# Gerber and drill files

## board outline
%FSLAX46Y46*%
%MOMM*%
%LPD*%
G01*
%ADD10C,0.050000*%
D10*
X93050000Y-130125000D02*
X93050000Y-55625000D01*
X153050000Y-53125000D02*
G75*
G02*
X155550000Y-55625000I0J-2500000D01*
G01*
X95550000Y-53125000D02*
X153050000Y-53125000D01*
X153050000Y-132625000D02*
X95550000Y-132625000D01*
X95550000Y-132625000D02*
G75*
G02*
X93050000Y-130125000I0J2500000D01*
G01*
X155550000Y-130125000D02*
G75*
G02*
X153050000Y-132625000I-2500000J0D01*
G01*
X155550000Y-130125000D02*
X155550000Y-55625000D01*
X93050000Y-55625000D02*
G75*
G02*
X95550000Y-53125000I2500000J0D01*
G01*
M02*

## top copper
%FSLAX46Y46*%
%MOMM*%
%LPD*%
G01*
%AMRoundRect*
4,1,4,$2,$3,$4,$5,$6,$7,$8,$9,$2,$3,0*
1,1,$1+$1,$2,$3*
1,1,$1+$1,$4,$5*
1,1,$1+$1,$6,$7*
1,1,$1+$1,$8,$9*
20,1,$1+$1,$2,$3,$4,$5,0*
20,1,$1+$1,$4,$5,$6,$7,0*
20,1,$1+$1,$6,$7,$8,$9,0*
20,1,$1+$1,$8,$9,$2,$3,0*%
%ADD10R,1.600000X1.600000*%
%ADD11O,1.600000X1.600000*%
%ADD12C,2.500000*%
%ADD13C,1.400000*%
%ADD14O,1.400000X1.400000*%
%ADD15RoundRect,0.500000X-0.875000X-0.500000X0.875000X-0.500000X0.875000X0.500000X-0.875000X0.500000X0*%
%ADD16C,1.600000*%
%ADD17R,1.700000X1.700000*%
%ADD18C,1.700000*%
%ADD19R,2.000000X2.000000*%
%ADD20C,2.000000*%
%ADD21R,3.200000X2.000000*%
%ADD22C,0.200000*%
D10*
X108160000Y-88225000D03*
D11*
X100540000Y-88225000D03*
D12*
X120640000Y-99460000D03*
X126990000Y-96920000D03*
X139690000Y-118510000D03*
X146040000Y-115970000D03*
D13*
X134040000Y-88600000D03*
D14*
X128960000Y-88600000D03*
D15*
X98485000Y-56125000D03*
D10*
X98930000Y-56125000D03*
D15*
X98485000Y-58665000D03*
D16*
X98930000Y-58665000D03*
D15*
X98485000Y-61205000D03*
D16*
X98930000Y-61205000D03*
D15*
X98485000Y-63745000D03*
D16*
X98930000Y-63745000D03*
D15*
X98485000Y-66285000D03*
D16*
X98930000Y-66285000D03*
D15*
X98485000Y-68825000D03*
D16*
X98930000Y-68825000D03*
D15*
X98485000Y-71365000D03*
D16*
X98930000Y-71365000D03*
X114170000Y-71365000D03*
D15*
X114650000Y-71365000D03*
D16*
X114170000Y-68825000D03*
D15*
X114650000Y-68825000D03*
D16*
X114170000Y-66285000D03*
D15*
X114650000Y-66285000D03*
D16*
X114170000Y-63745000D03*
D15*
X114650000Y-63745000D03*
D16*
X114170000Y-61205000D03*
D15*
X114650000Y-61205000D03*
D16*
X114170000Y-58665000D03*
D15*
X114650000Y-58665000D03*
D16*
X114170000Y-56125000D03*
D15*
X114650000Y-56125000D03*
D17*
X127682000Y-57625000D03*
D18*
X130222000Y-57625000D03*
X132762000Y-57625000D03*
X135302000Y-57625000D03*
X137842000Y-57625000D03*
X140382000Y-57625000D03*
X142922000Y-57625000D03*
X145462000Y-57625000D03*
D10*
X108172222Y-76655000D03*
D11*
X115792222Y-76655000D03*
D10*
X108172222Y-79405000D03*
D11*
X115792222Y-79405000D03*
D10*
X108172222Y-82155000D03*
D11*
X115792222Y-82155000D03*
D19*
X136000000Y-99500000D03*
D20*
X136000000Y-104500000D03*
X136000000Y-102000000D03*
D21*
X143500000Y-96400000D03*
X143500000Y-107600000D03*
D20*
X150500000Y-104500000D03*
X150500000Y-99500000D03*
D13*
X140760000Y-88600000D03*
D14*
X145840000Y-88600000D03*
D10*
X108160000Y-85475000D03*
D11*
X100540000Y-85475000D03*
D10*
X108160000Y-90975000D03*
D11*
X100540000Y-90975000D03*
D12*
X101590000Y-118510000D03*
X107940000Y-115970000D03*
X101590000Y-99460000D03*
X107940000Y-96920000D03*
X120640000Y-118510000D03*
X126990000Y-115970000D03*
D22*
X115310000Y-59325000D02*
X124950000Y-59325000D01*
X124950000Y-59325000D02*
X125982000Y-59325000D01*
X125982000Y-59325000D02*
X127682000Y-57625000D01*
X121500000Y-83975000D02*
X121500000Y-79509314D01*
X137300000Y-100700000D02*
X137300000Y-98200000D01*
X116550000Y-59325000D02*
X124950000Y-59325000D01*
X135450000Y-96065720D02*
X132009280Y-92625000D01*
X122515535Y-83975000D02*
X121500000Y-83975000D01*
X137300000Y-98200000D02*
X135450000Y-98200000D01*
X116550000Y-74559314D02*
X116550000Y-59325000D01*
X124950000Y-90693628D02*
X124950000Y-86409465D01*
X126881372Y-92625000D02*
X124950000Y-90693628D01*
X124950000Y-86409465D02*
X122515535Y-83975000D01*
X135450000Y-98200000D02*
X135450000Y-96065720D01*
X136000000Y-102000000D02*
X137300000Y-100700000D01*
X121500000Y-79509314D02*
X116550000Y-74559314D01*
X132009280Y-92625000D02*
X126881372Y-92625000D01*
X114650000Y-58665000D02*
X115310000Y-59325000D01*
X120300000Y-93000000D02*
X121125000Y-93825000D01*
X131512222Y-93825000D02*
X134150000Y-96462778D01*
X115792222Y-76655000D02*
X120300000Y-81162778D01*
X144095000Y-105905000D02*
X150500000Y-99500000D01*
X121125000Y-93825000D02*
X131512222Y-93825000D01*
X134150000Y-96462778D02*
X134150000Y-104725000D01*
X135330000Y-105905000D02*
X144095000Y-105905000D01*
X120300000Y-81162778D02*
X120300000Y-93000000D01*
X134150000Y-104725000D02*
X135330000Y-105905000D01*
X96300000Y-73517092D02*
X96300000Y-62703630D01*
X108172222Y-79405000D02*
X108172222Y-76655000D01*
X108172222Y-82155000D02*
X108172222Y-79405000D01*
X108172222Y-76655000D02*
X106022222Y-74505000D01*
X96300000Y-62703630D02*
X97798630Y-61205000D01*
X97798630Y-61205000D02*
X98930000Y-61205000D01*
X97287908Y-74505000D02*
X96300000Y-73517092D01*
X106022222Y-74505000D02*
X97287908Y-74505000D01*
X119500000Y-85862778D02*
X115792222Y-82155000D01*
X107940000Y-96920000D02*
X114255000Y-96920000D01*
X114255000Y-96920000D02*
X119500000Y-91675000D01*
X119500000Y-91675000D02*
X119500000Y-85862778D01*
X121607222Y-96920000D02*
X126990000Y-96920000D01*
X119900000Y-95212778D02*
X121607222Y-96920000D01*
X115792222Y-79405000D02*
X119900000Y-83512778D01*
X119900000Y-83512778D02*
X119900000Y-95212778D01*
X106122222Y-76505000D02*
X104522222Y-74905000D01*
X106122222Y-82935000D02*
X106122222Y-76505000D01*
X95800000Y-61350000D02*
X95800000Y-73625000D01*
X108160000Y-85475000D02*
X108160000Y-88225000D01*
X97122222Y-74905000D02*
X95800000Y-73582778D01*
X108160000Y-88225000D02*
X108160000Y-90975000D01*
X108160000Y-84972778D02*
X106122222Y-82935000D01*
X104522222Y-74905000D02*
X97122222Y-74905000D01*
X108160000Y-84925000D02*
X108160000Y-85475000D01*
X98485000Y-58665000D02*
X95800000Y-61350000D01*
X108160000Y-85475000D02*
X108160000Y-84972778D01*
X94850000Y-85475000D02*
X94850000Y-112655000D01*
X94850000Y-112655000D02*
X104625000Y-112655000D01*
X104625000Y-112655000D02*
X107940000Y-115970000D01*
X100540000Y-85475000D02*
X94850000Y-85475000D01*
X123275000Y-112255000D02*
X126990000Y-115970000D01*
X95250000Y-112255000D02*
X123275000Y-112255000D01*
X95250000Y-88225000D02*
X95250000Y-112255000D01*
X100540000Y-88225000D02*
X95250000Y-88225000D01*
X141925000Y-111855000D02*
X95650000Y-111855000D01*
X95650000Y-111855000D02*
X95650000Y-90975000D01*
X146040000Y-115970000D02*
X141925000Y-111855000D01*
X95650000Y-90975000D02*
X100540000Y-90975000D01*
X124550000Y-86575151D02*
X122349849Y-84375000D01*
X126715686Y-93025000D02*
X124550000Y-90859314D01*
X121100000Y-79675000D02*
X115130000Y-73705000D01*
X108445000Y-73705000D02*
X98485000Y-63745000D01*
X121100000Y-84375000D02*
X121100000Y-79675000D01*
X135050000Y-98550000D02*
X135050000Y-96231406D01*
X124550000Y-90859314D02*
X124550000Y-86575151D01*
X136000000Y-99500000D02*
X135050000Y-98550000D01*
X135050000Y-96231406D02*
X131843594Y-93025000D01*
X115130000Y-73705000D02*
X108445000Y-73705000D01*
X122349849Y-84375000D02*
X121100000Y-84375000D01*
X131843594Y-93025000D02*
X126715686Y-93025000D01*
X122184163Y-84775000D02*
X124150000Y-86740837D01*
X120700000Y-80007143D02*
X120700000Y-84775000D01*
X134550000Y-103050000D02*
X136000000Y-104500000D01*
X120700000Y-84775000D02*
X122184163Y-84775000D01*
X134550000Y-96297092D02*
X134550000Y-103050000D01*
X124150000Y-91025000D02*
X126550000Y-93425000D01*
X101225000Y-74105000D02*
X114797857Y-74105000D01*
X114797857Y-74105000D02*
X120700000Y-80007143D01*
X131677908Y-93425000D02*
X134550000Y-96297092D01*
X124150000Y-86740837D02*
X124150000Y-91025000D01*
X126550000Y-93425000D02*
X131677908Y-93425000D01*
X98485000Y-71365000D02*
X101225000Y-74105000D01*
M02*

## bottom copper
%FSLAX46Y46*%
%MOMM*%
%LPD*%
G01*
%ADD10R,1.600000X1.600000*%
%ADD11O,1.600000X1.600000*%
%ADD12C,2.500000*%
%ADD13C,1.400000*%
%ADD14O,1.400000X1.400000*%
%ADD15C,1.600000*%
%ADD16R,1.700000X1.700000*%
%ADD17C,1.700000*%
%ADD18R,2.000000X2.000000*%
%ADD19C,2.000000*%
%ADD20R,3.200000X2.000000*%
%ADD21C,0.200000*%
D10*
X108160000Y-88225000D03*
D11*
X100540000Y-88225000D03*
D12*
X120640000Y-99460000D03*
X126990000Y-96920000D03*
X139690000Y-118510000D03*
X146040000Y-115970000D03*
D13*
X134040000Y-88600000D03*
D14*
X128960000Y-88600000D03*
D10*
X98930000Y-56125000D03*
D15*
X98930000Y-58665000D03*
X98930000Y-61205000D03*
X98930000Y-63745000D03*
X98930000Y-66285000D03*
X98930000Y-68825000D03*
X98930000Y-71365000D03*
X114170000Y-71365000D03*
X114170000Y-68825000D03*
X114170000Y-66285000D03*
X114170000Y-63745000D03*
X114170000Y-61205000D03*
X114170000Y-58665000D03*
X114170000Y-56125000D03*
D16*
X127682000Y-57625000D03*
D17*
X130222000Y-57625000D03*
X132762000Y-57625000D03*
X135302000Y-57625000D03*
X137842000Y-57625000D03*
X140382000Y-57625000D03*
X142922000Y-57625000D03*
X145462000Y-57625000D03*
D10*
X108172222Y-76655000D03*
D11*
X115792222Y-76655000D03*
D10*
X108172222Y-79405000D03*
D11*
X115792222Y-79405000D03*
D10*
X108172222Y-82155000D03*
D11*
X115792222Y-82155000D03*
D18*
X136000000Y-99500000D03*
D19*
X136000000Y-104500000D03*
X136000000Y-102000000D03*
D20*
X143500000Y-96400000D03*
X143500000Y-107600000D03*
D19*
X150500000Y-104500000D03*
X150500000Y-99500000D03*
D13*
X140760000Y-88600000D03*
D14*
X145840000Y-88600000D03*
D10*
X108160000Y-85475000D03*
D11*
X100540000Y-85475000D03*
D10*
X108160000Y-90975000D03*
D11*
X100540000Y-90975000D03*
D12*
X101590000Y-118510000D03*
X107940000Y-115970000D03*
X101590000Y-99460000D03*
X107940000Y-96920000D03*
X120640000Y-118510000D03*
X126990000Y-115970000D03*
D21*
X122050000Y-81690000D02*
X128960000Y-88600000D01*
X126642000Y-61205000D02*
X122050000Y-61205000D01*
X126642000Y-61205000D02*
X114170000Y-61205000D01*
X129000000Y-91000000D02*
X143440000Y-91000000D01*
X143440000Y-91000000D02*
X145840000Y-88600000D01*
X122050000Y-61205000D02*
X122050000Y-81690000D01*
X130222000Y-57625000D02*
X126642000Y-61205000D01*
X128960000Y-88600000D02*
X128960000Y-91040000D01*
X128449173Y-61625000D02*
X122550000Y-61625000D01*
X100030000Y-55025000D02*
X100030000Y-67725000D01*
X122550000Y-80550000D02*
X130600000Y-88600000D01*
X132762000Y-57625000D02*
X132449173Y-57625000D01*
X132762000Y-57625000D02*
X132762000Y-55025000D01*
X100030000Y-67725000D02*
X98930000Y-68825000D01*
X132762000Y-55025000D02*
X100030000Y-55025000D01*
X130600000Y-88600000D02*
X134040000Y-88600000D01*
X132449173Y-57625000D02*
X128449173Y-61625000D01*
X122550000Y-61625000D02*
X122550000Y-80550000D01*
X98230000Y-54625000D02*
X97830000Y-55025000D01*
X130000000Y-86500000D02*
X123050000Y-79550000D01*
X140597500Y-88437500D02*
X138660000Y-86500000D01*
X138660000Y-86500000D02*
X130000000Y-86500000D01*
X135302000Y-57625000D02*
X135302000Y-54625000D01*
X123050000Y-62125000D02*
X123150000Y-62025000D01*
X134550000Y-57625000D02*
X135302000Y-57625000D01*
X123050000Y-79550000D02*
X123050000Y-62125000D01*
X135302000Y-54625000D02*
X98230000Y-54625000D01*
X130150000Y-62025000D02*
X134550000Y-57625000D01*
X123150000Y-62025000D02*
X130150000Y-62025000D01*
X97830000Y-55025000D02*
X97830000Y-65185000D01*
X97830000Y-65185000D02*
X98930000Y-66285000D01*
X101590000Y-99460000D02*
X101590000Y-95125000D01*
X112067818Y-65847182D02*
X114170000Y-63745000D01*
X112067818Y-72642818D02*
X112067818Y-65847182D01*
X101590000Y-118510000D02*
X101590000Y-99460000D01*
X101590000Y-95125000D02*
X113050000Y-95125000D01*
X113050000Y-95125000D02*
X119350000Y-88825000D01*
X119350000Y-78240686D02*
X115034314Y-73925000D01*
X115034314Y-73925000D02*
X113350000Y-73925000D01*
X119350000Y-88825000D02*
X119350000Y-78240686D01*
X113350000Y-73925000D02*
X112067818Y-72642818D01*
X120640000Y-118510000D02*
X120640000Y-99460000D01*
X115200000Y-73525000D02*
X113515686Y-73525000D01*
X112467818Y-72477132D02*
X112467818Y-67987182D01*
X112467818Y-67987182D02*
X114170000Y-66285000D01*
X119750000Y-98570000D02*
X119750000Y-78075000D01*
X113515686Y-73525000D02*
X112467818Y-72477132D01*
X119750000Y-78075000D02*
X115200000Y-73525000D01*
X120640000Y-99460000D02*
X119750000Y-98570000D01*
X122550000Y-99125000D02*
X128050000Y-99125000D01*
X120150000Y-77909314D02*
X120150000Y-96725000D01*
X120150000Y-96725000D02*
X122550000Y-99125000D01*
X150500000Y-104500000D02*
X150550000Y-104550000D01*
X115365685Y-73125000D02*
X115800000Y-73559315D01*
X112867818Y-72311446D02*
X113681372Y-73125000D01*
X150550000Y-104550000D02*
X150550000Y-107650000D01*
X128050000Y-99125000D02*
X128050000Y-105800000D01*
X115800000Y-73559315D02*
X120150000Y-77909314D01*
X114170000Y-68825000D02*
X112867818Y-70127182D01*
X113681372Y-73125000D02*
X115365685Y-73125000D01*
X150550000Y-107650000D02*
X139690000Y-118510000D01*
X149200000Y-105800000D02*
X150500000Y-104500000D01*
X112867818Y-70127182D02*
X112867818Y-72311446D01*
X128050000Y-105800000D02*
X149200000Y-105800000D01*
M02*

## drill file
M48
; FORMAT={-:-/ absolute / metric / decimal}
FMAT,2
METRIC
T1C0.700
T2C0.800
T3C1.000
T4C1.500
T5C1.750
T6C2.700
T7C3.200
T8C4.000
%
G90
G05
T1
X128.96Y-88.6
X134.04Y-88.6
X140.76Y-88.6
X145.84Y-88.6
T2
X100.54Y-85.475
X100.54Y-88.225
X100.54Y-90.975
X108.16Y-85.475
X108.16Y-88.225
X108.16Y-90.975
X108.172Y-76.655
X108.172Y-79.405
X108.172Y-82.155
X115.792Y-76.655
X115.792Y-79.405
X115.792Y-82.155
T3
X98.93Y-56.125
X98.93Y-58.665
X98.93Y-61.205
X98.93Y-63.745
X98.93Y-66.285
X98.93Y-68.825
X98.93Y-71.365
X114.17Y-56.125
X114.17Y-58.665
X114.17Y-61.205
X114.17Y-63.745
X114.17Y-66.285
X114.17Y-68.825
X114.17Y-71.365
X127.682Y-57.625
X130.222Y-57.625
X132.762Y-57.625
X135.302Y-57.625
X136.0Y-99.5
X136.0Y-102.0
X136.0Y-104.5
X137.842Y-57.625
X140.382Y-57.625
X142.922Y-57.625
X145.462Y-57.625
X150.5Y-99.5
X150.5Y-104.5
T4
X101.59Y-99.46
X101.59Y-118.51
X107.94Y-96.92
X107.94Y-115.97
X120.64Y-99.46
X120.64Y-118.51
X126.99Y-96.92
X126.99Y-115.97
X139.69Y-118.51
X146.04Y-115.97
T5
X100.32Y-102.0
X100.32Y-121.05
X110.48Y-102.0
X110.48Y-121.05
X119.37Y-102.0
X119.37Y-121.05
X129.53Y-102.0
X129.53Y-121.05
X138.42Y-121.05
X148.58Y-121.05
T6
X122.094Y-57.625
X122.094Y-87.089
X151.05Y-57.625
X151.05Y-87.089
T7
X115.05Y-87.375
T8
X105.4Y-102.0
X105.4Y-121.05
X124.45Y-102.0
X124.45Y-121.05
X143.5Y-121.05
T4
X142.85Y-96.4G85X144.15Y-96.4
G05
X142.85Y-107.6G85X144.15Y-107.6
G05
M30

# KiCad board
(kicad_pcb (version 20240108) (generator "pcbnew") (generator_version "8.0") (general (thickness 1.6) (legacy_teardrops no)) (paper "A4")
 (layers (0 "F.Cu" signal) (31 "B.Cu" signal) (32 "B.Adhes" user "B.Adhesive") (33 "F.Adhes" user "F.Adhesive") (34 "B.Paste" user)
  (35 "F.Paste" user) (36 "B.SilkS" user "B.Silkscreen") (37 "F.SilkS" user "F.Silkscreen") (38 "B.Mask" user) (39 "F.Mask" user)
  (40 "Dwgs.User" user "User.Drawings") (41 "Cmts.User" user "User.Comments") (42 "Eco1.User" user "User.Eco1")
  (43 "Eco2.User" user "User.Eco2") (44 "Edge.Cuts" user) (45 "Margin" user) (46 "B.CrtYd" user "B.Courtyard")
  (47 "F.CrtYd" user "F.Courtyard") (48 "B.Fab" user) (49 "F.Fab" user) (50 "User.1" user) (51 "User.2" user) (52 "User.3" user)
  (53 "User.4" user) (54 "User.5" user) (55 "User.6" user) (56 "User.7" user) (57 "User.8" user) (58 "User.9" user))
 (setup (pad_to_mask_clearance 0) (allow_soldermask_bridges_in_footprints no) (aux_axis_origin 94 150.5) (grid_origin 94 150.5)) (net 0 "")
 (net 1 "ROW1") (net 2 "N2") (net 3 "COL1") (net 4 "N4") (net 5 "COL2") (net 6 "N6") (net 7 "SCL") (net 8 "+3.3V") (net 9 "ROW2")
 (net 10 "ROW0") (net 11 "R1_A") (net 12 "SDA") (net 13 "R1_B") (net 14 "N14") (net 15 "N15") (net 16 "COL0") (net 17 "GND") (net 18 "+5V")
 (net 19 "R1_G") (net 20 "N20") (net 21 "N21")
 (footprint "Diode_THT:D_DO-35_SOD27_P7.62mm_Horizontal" (layer "F.Cu") (at 108.16 88.225 180)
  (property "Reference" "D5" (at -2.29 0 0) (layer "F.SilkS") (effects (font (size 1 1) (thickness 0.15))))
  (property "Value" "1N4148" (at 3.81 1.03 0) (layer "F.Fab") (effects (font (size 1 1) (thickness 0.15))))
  (pad "1" thru_hole rect (at 0 0 180) (size 1.6 1.6) (drill 0.8) (layers "*.Cu" "*.Mask") (remove_unused_layers no) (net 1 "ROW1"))
  (pad "2" thru_hole oval (at 7.62 0 180) (size 1.6 1.6) (drill 0.8) (layers "*.Cu" "*.Mask") (remove_unused_layers no) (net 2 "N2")))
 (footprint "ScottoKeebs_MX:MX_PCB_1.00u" (layer "F.Cu") (at 124.45 102)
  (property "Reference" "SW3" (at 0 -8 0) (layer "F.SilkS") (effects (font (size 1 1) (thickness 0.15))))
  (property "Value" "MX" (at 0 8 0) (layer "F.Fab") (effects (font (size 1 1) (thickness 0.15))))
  (pad "" np_thru_hole circle (at -5.08 0) (size 1.75 1.75) (drill 1.75) (layers "*.Cu" "*.Mask"))
  (pad "" np_thru_hole circle (at 0 0) (size 4 4) (drill 4) (layers "*.Cu" "*.Mask"))
  (pad "" np_thru_hole circle (at 5.08 0) (size 1.75 1.75) (drill 1.75) (layers "*.Cu" "*.Mask"))
  (pad "1" thru_hole circle (at -3.81 -2.54) (size 2.5 2.5) (drill 1.5) (layers "*.Cu" "*.Mask") (remove_unused_layers no) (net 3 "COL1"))
  (pad "2" thru_hole circle (at 2.54 -5.08) (size 2.5 2.5) (drill 1.5) (layers "*.Cu" "*.Mask") (remove_unused_layers no) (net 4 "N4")))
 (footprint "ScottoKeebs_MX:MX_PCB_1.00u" (layer "F.Cu") (at 143.5 121.05)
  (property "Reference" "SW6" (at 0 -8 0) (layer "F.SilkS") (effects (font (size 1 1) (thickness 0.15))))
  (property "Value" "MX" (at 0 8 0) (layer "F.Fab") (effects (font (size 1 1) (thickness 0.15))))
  (pad "" np_thru_hole circle (at -5.08 0) (size 1.75 1.75) (drill 1.75) (layers "*.Cu" "*.Mask"))
  (pad "" np_thru_hole circle (at 0 0) (size 4 4) (drill 4) (layers "*.Cu" "*.Mask"))
  (pad "" np_thru_hole circle (at 5.08 0) (size 1.75 1.75) (drill 1.75) (layers "*.Cu" "*.Mask"))
  (pad "1" thru_hole circle (at -3.81 -2.54) (size 2.5 2.5) (drill 1.5) (layers "*.Cu" "*.Mask") (remove_unused_layers no) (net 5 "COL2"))
  (pad "2" thru_hole circle (at 2.54 -5.08) (size 2.5 2.5) (drill 1.5) (layers "*.Cu" "*.Mask") (remove_unused_layers no) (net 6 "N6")))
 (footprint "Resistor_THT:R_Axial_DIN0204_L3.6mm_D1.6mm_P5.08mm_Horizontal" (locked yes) (layer "F.Cu") (at 134.04 88.6 180)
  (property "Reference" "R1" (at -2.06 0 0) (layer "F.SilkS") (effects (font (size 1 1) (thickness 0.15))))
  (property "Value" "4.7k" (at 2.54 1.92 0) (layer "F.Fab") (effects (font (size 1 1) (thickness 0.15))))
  (pad "1" thru_hole circle (at 0 0 180) (size 1.4 1.4) (drill 0.7) (layers "*.Cu" "*.Mask") (remove_unused_layers no) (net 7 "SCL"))
  (pad "2" thru_hole oval (at 5.08 0 180) (size 1.4 1.4) (drill 0.7) (layers "*.Cu" "*.Mask") (remove_unused_layers no) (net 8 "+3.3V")))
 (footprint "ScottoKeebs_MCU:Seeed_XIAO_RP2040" (layer "F.Cu") (at 106.55 63.745)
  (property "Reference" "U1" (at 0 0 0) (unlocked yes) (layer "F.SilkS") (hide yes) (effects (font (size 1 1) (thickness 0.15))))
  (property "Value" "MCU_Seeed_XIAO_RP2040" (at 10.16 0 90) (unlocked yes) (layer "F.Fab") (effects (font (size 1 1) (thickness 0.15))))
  (pad "1" smd roundrect (at -8.065 -7.62) (size 2.75 2) (layers "F.Cu" "F.Paste" "F.Mask") (roundrect_rratio 0.25) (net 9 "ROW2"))
  (pad "1" thru_hole rect (at -7.62 -7.62 90) (size 1.6 1.6) (drill 1) (layers "*.Cu" "*.Mask") (remove_unused_layers no) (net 9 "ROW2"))
  (pad "2" smd roundrect (at -8.065 -5.08) (size 2.75 2) (layers "F.Cu" "F.Paste" "F.Mask") (roundrect_rratio 0.25) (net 1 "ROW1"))
  (pad "2" thru_hole circle (at -7.62 -5.08 90) (size 1.6 1.6) (drill 1) (layers "*.Cu" "*.Mask") (remove_unused_layers no) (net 1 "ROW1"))
  (pad "3" smd roundrect (at -8.065 -2.54) (size 2.75 2) (layers "F.Cu" "F.Paste" "F.Mask") (roundrect_rratio 0.25) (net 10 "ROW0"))
  (pad "3" thru_hole circle (at -7.62 -2.54 90) (size 1.6 1.6) (drill 1) (layers "*.Cu" "*.Mask") (remove_unused_layers no) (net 10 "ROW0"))
  (pad "4" smd roundrect (at -8.065 0) (size 2.75 2) (layers "F.Cu" "F.Paste" "F.Mask") (roundrect_rratio 0.25) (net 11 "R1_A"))
  (pad "4" thru_hole circle (at -7.62 0 90) (size 1.6 1.6) (drill 1) (layers "*.Cu" "*.Mask") (remove_unused_layers no) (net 11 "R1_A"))
  (pad "5" smd roundrect (at -8.065 2.54) (size 2.75 2) (layers "F.Cu" "F.Paste" "F.Mask") (roundrect_rratio 0.25) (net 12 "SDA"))
  (pad "5" thru_hole circle (at -7.62 2.54 90) (size 1.6 1.6) (drill 1) (layers "*.Cu" "*.Mask") (remove_unused_layers no) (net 12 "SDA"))
  (pad "6" smd roundrect (at -8.065 5.08) (size 2.75 2) (layers "F.Cu" "F.Paste" "F.Mask") (roundrect_rratio 0.25) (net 7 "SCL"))
  (pad "6" thru_hole circle (at -7.62 5.08 90) (size 1.6 1.6) (drill 1) (layers "*.Cu" "*.Mask") (remove_unused_layers no) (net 7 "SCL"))
  (pad "7" smd roundrect (at -8.065 7.62) (size 2.75 2) (layers "F.Cu" "F.Paste" "F.Mask") (roundrect_rratio 0.25) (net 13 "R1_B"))
  (pad "7" thru_hole circle (at -7.62 7.62 90) (size 1.6 1.6) (drill 1) (layers "*.Cu" "*.Mask") (remove_unused_layers no) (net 13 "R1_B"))
  (pad "8" thru_hole circle (at 7.62 7.62 90) (size 1.6 1.6) (drill 1) (layers "*.Cu" "*.Mask") (remove_unused_layers no) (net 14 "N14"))
  (pad "8" smd roundrect (at 8.1 7.62) (size 2.75 2) (layers "F.Cu" "F.Paste" "F.Mask") (roundrect_rratio 0.25) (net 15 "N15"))
  (pad "9" thru_hole circle (at 7.62 5.08 90) (size 1.6 1.6) (drill 1) (layers "*.Cu" "*.Mask") (remove_unused_layers no) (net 5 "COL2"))
  (pad "9" smd roundrect (at 8.1 5.08) (size 2.75 2) (layers "F.Cu" "F.Paste" "F.Mask") (roundrect_rratio 0.25) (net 5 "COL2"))
  (pad "10" thru_hole circle (at 7.62 2.54 90) (size 1.6 1.6) (drill 1) (layers "*.Cu" "*.Mask") (remove_unused_layers no) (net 3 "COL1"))
  (pad "10" smd roundrect (at 8.1 2.54) (size 2.75 2) (layers "F.Cu" "F.Paste" "F.Mask") (roundrect_rratio 0.25) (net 3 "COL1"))
  (pad "11" thru_hole circle (at 7.62 0 90) (size 1.6 1.6) (drill 1) (layers "*.Cu" "*.Mask") (remove_unused_layers no) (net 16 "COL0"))
  (pad "11" smd roundrect (at 8.1 0) (size 2.75 2) (layers "F.Cu" "F.Paste" "F.Mask") (roundrect_rratio 0.25) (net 16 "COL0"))
  (pad "12" thru_hole circle (at 7.62 -2.54 90) (size 1.6 1.6) (drill 1) (layers "*.Cu" "*.Mask") (remove_unused_layers no) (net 8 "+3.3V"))
  (pad "12" smd roundrect (at 8.1 -2.54) (size 2.75 2) (layers "F.Cu" "F.Paste" "F.Mask") (roundrect_rratio 0.25) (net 8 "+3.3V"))
  (pad "13" thru_hole circle (at 7.62 -5.08 90) (size 1.6 1.6) (drill 1) (layers "*.Cu" "*.Mask") (remove_unused_layers no) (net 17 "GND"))
  (pad "13" smd roundrect (at 8.1 -5.08) (size 2.75 2) (layers "F.Cu" "F.Paste" "F.Mask") (roundrect_rratio 0.25) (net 17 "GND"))
  (pad "14" thru_hole circle (at 7.62 -7.62 90) (size 1.6 1.6) (drill 1) (layers "*.Cu" "*.Mask") (remove_unused_layers no) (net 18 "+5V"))
  (pad "14" smd roundrect (at 8.1 -7.62) (size 2.75 2) (layers "F.Cu" "F.Paste" "F.Mask") (roundrect_rratio 0.25) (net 18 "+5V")))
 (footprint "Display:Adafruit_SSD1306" (layer "F.Cu") (at 127.682 57.625)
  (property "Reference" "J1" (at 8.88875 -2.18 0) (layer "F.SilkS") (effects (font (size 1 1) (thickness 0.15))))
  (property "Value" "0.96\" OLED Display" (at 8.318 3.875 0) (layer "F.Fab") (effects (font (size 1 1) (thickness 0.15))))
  (pad "" np_thru_hole circle (at -5.588 0) (size 2.7 2.7) (drill 2.7) (layers "*.Cu" "*.Mask"))
  (pad "" np_thru_hole circle (at -5.588 29.464) (size 2.7 2.7) (drill 2.7) (layers "*.Cu" "*.Mask"))
  (pad "" np_thru_hole circle (at 23.368 0) (size 2.7 2.7) (drill 2.7) (layers "*.Cu" "*.Mask"))
  (pad "" np_thru_hole circle (at 23.368 29.464) (size 2.7 2.7) (drill 2.7) (layers "*.Cu" "*.Mask"))
  (pad "1" thru_hole rect (at 0 0) (size 1.7 1.7) (drill 1) (layers "*.Cu" "*.Mask") (remove_unused_layers no) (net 17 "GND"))
  (pad "2" thru_hole circle (at 2.54 0) (size 1.7 1.7) (drill 1) (layers "*.Cu" "*.Mask") (remove_unused_layers no) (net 8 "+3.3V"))
  (pad "3" thru_hole circle (at 5.08 0) (size 1.7 1.7) (drill 1) (layers "*.Cu" "*.Mask") (remove_unused_layers no) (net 7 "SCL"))
  (pad "4" thru_hole circle (at 7.62 0) (size 1.7 1.7) (drill 1) (layers "*.Cu" "*.Mask") (remove_unused_layers no) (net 12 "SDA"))
  (pad "5" thru_hole circle (at 10.16 0) (size 1.7 1.7) (drill 1) (layers "*.Cu" "*.Mask") (remove_unused_layers no))
  (pad "6" thru_hole circle (at 12.7 0) (size 1.7 1.7) (drill 1) (layers "*.Cu" "*.Mask") (remove_unused_layers no))
  (pad "7" thru_hole circle (at 15.24 0) (size 1.7 1.7) (drill 1) (layers "*.Cu" "*.Mask") (remove_unused_layers no))
  (pad "8" thru_hole circle (at 17.78 0) (size 1.7 1.7) (drill 1) (layers "*.Cu" "*.Mask") (remove_unused_layers no)))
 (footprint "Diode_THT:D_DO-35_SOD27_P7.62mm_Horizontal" (layer "F.Cu") (at 108.172222 76.655)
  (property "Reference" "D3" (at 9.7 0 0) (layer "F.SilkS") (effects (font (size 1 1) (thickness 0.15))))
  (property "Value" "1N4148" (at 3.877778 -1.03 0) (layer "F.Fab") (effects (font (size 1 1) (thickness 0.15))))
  (pad "1" thru_hole rect (at 0 0) (size 1.6 1.6) (drill 0.8) (layers "*.Cu" "*.Mask") (remove_unused_layers no) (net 10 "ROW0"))
  (pad "2" thru_hole oval (at 7.62 0) (size 1.6 1.6) (drill 0.8) (layers "*.Cu" "*.Mask") (remove_unused_layers no) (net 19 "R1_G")))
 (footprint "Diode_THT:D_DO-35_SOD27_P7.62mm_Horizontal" (layer "F.Cu") (at 108.172222 79.405)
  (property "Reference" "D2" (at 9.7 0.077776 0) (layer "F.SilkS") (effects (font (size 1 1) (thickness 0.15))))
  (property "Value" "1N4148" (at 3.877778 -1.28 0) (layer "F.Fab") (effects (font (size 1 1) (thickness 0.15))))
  (pad "1" thru_hole rect (at 0 0) (size 1.6 1.6) (drill 0.8) (layers "*.Cu" "*.Mask") (remove_unused_layers no) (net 10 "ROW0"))
  (pad "2" thru_hole oval (at 7.62 0) (size 1.6 1.6) (drill 0.8) (layers "*.Cu" "*.Mask") (remove_unused_layers no) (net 4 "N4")))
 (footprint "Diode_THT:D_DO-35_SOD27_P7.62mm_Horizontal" (layer "F.Cu") (at 108.172222 82.155)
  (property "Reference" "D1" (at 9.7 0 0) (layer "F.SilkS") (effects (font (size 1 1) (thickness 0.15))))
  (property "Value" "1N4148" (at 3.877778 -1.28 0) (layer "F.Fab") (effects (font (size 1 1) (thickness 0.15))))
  (pad "1" thru_hole rect (at 0 0) (size 1.6 1.6) (drill 0.8) (layers "*.Cu" "*.Mask") (remove_unused_layers no) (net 10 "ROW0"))
  (pad "2" thru_hole oval (at 7.62 0) (size 1.6 1.6) (drill 0.8) (layers "*.Cu" "*.Mask") (remove_unused_layers no) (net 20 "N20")))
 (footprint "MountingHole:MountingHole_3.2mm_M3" (layer "F.Cu") (at 115.05 87.375)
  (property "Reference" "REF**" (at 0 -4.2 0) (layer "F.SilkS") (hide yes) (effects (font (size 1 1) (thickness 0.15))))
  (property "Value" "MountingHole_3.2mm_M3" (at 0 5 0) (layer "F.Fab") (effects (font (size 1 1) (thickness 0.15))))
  (pad "" np_thru_hole circle (at 0 0) (size 3.2 3.2) (drill 3.2) (layers "F&B.Cu" "*.Mask")))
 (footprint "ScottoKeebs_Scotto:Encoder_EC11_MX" (layer "F.Cu") (at 143.5 102)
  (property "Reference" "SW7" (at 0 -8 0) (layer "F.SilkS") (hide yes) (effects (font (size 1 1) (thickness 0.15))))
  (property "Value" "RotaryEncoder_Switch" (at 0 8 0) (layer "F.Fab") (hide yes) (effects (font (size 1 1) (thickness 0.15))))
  (pad "A" thru_hole rect (at -7.5 -2.5) (size 2 2) (drill 1) (layers "*.Cu" "*.Mask") (remove_unused_layers no) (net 11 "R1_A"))
  (pad "B" thru_hole circle (at -7.5 2.5) (size 2 2) (drill 1) (layers "*.Cu" "*.Mask") (remove_unused_layers no) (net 13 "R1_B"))
  (pad "C" thru_hole circle (at -7.5 0) (size 2 2) (drill 1) (layers "*.Cu" "*.Mask") (remove_unused_layers no) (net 17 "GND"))
  (pad "MP" thru_hole rect (at 0 -5.6) (size 3.2 2) (drill oval 2.8 1.5) (layers "*.Cu" "*.Mask") (remove_unused_layers no))
  (pad "MP" thru_hole rect (at 0 5.6) (size 3.2 2) (drill oval 2.8 1.5) (layers "*.Cu" "*.Mask") (remove_unused_layers no))
  (pad "S1" thru_hole circle (at 7 2.5) (size 2 2) (drill 1) (layers "*.Cu" "*.Mask") (remove_unused_layers no) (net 5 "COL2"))
  (pad "S2" thru_hole circle (at 7 -2.5) (size 2 2) (drill 1) (layers "*.Cu" "*.Mask") (remove_unused_layers no) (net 19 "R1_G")))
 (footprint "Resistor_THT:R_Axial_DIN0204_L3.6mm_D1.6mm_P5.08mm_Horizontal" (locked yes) (layer "F.Cu") (at 140.76 88.6)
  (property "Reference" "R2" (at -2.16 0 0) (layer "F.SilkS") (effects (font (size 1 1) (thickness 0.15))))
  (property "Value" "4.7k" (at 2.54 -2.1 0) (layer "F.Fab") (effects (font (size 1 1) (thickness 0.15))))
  (pad "1" thru_hole circle (at 0 0) (size 1.4 1.4) (drill 0.7) (layers "*.Cu" "*.Mask") (remove_unused_layers no) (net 12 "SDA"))
  (pad "2" thru_hole oval (at 5.08 0) (size 1.4 1.4) (drill 0.7) (layers "*.Cu" "*.Mask") (remove_unused_layers no) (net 8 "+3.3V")))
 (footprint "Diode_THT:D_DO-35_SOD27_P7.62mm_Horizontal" (layer "F.Cu") (at 108.16 85.475 180)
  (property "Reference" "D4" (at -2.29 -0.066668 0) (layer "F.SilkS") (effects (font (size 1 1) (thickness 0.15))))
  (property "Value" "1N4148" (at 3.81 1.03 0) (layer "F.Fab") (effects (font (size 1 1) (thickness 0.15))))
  (pad "1" thru_hole rect (at 0 0 180) (size 1.6 1.6) (drill 0.8) (layers "*.Cu" "*.Mask") (remove_unused_layers no) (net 1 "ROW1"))
  (pad "2" thru_hole oval (at 7.62 0 180) (size 1.6 1.6) (drill 0.8) (layers "*.Cu" "*.Mask") (remove_unused_layers no) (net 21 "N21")))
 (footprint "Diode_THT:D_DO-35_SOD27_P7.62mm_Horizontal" (layer "F.Cu") (at 108.16 90.975 180)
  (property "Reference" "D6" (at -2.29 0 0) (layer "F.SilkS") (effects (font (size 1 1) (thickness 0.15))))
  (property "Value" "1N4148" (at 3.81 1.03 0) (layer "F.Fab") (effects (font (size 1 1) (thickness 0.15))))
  (pad "1" thru_hole rect (at 0 0 180) (size 1.6 1.6) (drill 0.8) (layers "*.Cu" "*.Mask") (remove_unused_layers no) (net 1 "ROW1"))
  (pad "2" thru_hole oval (at 7.62 0 180) (size 1.6 1.6) (drill 0.8) (layers "*.Cu" "*.Mask") (remove_unused_layers no) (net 6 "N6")))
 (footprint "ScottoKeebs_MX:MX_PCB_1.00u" (layer "F.Cu") (at 105.4 121.05)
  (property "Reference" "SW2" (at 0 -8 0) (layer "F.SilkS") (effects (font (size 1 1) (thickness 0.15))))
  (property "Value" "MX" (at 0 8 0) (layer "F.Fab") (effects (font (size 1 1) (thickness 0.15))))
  (pad "" np_thru_hole circle (at -5.08 0) (size 1.75 1.75) (drill 1.75) (layers "*.Cu" "*.Mask"))
  (pad "" np_thru_hole circle (at 0 0) (size 4 4) (drill 4) (layers "*.Cu" "*.Mask"))
  (pad "" np_thru_hole circle (at 5.08 0) (size 1.75 1.75) (drill 1.75) (layers "*.Cu" "*.Mask"))
  (pad "1" thru_hole circle (at -3.81 -2.54) (size 2.5 2.5) (drill 1.5) (layers "*.Cu" "*.Mask") (remove_unused_layers no) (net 16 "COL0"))
  (pad "2" thru_hole circle (at 2.54 -5.08) (size 2.5 2.5) (drill 1.5) (layers "*.Cu" "*.Mask") (remove_unused_layers no) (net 21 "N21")))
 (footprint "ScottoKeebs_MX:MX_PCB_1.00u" (layer "F.Cu") (at 105.4 102)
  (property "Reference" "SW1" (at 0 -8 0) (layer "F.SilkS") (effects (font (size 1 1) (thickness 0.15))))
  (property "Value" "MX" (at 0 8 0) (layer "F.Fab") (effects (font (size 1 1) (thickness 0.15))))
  (pad "" np_thru_hole circle (at -5.08 0) (size 1.75 1.75) (drill 1.75) (layers "*.Cu" "*.Mask"))
  (pad "" np_thru_hole circle (at 0 0) (size 4 4) (drill 4) (layers "*.Cu" "*.Mask"))
  (pad "" np_thru_hole circle (at 5.08 0) (size 1.75 1.75) (drill 1.75) (layers "*.Cu" "*.Mask"))
  (pad "1" thru_hole circle (at -3.81 -2.54) (size 2.5 2.5) (drill 1.5) (layers "*.Cu" "*.Mask") (remove_unused_layers no) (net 16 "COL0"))
  (pad "2" thru_hole circle (at 2.54 -5.08) (size 2.5 2.5) (drill 1.5) (layers "*.Cu" "*.Mask") (remove_unused_layers no) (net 20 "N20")))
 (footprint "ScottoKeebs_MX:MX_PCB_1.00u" (layer "F.Cu") (at 124.45 121.05)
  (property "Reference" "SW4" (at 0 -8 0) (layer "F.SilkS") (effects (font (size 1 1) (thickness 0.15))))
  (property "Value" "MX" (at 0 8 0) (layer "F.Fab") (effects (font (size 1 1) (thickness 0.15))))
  (pad "" np_thru_hole circle (at -5.08 0) (size 1.75 1.75) (drill 1.75) (layers "*.Cu" "*.Mask"))
  (pad "" np_thru_hole circle (at 0 0) (size 4 4) (drill 4) (layers "*.Cu" "*.Mask"))
  (pad "" np_thru_hole circle (at 5.08 0) (size 1.75 1.75) (drill 1.75) (layers "*.Cu" "*.Mask"))
  (pad "1" thru_hole circle (at -3.81 -2.54) (size 2.5 2.5) (drill 1.5) (layers "*.Cu" "*.Mask") (remove_unused_layers no) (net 3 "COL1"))
  (pad "2" thru_hole circle (at 2.54 -5.08) (size 2.5 2.5) (drill 1.5) (layers "*.Cu" "*.Mask") (remove_unused_layers no) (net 2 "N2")))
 (gr_line (start 93.05 130.125) (end 93.05 55.625) (stroke (width 0.05) (type default)) (layer "Edge.Cuts"))
 (gr_arc (start 153.05 53.125) (mid 154.817767 53.857233) (end 155.55 55.625) (stroke (width 0.05) (type default)) (layer "Edge.Cuts"))
 (gr_line (start 95.55 53.125) (end 153.05 53.125) (stroke (width 0.05) (type default)) (layer "Edge.Cuts"))
 (gr_line (start 153.05 132.625) (end 95.55 132.625) (stroke (width 0.05) (type default)) (layer "Edge.Cuts"))
 (gr_arc (start 95.55 132.625) (mid 93.782233 131.892767) (end 93.05 130.125) (stroke (width 0.05) (type default)) (layer "Edge.Cuts"))
 (gr_arc (start 155.55 130.125) (mid 154.817767 131.892767) (end 153.05 132.625) (stroke (width 0.05) (type default)) (layer "Edge.Cuts"))
 (gr_line (start 155.55 130.125) (end 155.55 55.625) (stroke (width 0.05) (type default)) (layer "Edge.Cuts"))
 (gr_arc (start 93.05 55.625) (mid 93.782233 53.857233) (end 95.55 53.125) (stroke (width 0.05) (type default)) (layer "Edge.Cuts"))
 (segment (start 115.31 59.325) (end 124.95 59.325) (width 0.2) (layer "F.Cu") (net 17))
 (segment (start 124.95 59.325) (end 125.982 59.325) (width 0.2) (layer "F.Cu") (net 17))
 (segment (start 125.982 59.325) (end 127.682 57.625) (width 0.2) (layer "F.Cu") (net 17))
 (segment (start 121.5 83.975) (end 121.5 79.509314) (width 0.2) (layer "F.Cu") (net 17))
 (segment (start 137.3 100.7) (end 137.3 98.2) (width 0.2) (layer "F.Cu") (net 17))
 (segment (start 116.55 59.325) (end 124.95 59.325) (width 0.2) (layer "F.Cu") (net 17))
 (segment (start 135.45 96.06572) (end 132.00928 92.625) (width 0.2) (layer "F.Cu") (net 17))
 (segment (start 122.515535 83.975) (end 121.5 83.975) (width 0.2) (layer "F.Cu") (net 17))
 (segment (start 137.3 98.2) (end 135.45 98.2) (width 0.2) (layer "F.Cu") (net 17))
 (segment (start 116.55 74.559314) (end 116.55 59.325) (width 0.2) (layer "F.Cu") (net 17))
 (segment (start 124.95 90.693628) (end 124.95 86.409465) (width 0.2) (layer "F.Cu") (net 17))
 (segment (start 126.881372 92.625) (end 124.95 90.693628) (width 0.2) (layer "F.Cu") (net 17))
 (segment (start 124.95 86.409465) (end 122.515535 83.975) (width 0.2) (layer "F.Cu") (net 17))
 (segment (start 135.45 98.2) (end 135.45 96.06572) (width 0.2) (layer "F.Cu") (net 17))
 (segment (start 136 102) (end 137.3 100.7) (width 0.2) (layer "F.Cu") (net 17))
 (segment (start 121.5 79.509314) (end 116.55 74.559314) (width 0.2) (layer "F.Cu") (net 17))
 (segment (start 132.00928 92.625) (end 126.881372 92.625) (width 0.2) (layer "F.Cu") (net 17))
 (segment (start 114.65 58.665) (end 115.31 59.325) (width 0.2) (layer "F.Cu") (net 17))
 (segment (start 120.3 93) (end 121.125 93.825) (width 0.2) (layer "F.Cu") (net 19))
 (segment (start 131.512222 93.825) (end 134.15 96.462778) (width 0.2) (layer "F.Cu") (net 19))
 (segment (start 115.792222 76.655) (end 120.3 81.162778) (width 0.2) (layer "F.Cu") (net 19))
 (segment (start 144.095 105.905) (end 150.5 99.5) (width 0.2) (layer "F.Cu") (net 19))
 (segment (start 121.125 93.825) (end 131.512222 93.825) (width 0.2) (layer "F.Cu") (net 19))
 (segment (start 134.15 96.462778) (end 134.15 104.725) (width 0.2) (layer "F.Cu") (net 19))
 (segment (start 135.33 105.905) (end 144.095 105.905) (width 0.2) (layer "F.Cu") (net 19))
 (segment (start 120.3 81.162778) (end 120.3 93) (width 0.2) (layer "F.Cu") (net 19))
 (segment (start 134.15 104.725) (end 135.33 105.905) (width 0.2) (layer "F.Cu") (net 19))
 (segment (start 96.3 73.517092) (end 96.3 62.70363) (width 0.2) (layer "F.Cu") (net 10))
 (segment (start 108.172222 79.405) (end 108.172222 76.655) (width 0.2) (layer "F.Cu") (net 10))
 (segment (start 108.172222 82.155) (end 108.172222 79.405) (width 0.2) (layer "F.Cu") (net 10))
 (segment (start 108.172222 76.655) (end 106.022222 74.505) (width 0.2) (layer "F.Cu") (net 10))
 (segment (start 96.3 62.70363) (end 97.79863 61.205) (width 0.2) (layer "F.Cu") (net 10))
 (segment (start 97.79863 61.205) (end 98.93 61.205) (width 0.2) (layer "F.Cu") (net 10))
 (segment (start 97.287908 74.505) (end 96.3 73.517092) (width 0.2) (layer "F.Cu") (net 10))
 (segment (start 106.022222 74.505) (end 97.287908 74.505) (width 0.2) (layer "F.Cu") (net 10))
 (segment (start 119.5 85.862778) (end 115.792222 82.155) (width 0.2) (layer "F.Cu") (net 20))
 (segment (start 107.94 96.92) (end 114.255 96.92) (width 0.2) (layer "F.Cu") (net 20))
 (segment (start 114.255 96.92) (end 119.5 91.675) (width 0.2) (layer "F.Cu") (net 20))
 (segment (start 119.5 91.675) (end 119.5 85.862778) (width 0.2) (layer "F.Cu") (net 20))
 (segment (start 121.607222 96.92) (end 126.99 96.92) (width 0.2) (layer "F.Cu") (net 4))
 (segment (start 119.9 95.212778) (end 121.607222 96.92) (width 0.2) (layer "F.Cu") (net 4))
 (segment (start 115.792222 79.405) (end 119.9 83.512778) (width 0.2) (layer "F.Cu") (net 4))
 (segment (start 119.9 83.512778) (end 119.9 95.212778) (width 0.2) (layer "F.Cu") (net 4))
 (segment (start 106.122222 76.505) (end 104.522222 74.905) (width 0.2) (layer "F.Cu") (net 1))
 (segment (start 106.122222 82.935) (end 106.122222 76.505) (width 0.2) (layer "F.Cu") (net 1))
 (segment (start 95.8 61.35) (end 95.8 73.625) (width 0.2) (layer "F.Cu") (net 1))
 (segment (start 108.16 85.475) (end 108.16 88.225) (width 0.2) (layer "F.Cu") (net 1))
 (segment (start 97.122222 74.905) (end 95.8 73.582778) (width 0.2) (layer "F.Cu") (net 1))
 (segment (start 108.16 88.225) (end 108.16 90.975) (width 0.2) (layer "F.Cu") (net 1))
 (segment (start 108.16 84.972778) (end 106.122222 82.935) (width 0.2) (layer "F.Cu") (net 1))
 (segment (start 104.522222 74.905) (end 97.122222 74.905) (width 0.2) (layer "F.Cu") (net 1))
 (segment (start 108.16 84.925) (end 108.16 85.475) (width 0.2) (layer "F.Cu") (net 1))
 (segment (start 98.485 58.665) (end 95.8 61.35) (width 0.2) (layer "F.Cu") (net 1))
 (segment (start 108.16 85.475) (end 108.16 84.972778) (width 0.2) (layer "F.Cu") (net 1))
 (segment (start 94.85 85.475) (end 94.85 112.655) (width 0.2) (layer "F.Cu") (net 21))
 (segment (start 94.85 112.655) (end 104.625 112.655) (width 0.2) (layer "F.Cu") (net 21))
 (segment (start 104.625 112.655) (end 107.94 115.97) (width 0.2) (layer "F.Cu") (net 21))
 (segment (start 100.54 85.475) (end 94.85 85.475) (width 0.2) (layer "F.Cu") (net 21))
 (segment (start 123.275 112.255) (end 126.99 115.97) (width 0.2) (layer "F.Cu") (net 2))
 (segment (start 95.25 112.255) (end 123.275 112.255) (width 0.2) (layer "F.Cu") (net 2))
 (segment (start 95.25 88.225) (end 95.25 112.255) (width 0.2) (layer "F.Cu") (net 2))
 (segment (start 100.54 88.225) (end 95.25 88.225) (width 0.2) (layer "F.Cu") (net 2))
 (segment (start 141.925 111.855) (end 95.65 111.855) (width 0.2) (layer "F.Cu") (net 6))
 (segment (start 95.65 111.855) (end 95.65 90.975) (width 0.2) (layer "F.Cu") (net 6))
 (segment (start 146.04 115.97) (end 141.925 111.855) (width 0.2) (layer "F.Cu") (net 6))
 (segment (start 95.65 90.975) (end 100.54 90.975) (width 0.2) (layer "F.Cu") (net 6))
 (segment (start 124.55 86.575151) (end 122.349849 84.375) (width 0.2) (layer "F.Cu") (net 11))
 (segment (start 126.715686 93.025) (end 124.55 90.859314) (width 0.2) (layer "F.Cu") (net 11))
 (segment (start 121.1 79.675) (end 115.13 73.705) (width 0.2) (layer "F.Cu") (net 11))
 (segment (start 108.445 73.705) (end 98.485 63.745) (width 0.2) (layer "F.Cu") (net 11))
 (segment (start 121.1 84.375) (end 121.1 79.675) (width 0.2) (layer "F.Cu") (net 11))
 (segment (start 135.05 98.55) (end 135.05 96.231406) (width 0.2) (layer "F.Cu") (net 11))
 (segment (start 124.55 90.859314) (end 124.55 86.575151) (width 0.2) (layer "F.Cu") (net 11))
 (segment (start 136 99.5) (end 135.05 98.55) (width 0.2) (layer "F.Cu") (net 11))
 (segment (start 135.05 96.231406) (end 131.843594 93.025) (width 0.2) (layer "F.Cu") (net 11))
 (segment (start 115.13 73.705) (end 108.445 73.705) (width 0.2) (layer "F.Cu") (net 11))
 (segment (start 122.349849 84.375) (end 121.1 84.375) (width 0.2) (layer "F.Cu") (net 11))
 (segment (start 131.843594 93.025) (end 126.715686 93.025) (width 0.2) (layer "F.Cu") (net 11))
 (segment (start 122.05 81.69) (end 128.96 88.6) (width 0.2) (layer "B.Cu") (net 8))
 (segment (start 126.642 61.205) (end 122.05 61.205) (width 0.2) (layer "B.Cu") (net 8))
 (segment (start 126.642 61.205) (end 114.17 61.205) (width 0.2) (layer "B.Cu") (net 8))
 (segment (start 129 91) (end 143.44 91) (width 0.2) (layer "B.Cu") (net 8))
 (segment (start 143.44 91) (end 145.84 88.6) (width 0.2) (layer "B.Cu") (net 8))
 (segment (start 122.05 61.205) (end 122.05 81.69) (width 0.2) (layer "B.Cu") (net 8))
 (segment (start 130.222 57.625) (end 126.642 61.205) (width 0.2) (layer "B.Cu") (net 8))
 (segment (start 128.96 88.6) (end 128.96 91.04) (width 0.2) (layer "B.Cu") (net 8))
 (segment (start 128.449173 61.625) (end 122.55 61.625) (width 0.2) (layer "B.Cu") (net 7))
 (segment (start 100.03 55.025) (end 100.03 67.725) (width 0.2) (layer "B.Cu") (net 7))
 (segment (start 122.55 80.55) (end 130.6 88.6) (width 0.2) (layer "B.Cu") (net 7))
 (segment (start 132.762 57.625) (end 132.449173 57.625) (width 0.2) (layer "B.Cu") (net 7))
 (segment (start 132.762 57.625) (end 132.762 55.025) (width 0.2) (layer "B.Cu") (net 7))
 (segment (start 100.03 67.725) (end 98.93 68.825) (width 0.2) (layer "B.Cu") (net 7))
 (segment (start 132.762 55.025) (end 100.03 55.025) (width 0.2) (layer "B.Cu") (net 7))
 (segment (start 130.6 88.6) (end 134.04 88.6) (width 0.2) (layer "B.Cu") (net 7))
 (segment (start 132.449173 57.625) (end 128.449173 61.625) (width 0.2) (layer "B.Cu") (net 7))
 (segment (start 122.55 61.625) (end 122.55 80.55) (width 0.2) (layer "B.Cu") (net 7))
 (segment (start 98.23 54.625) (end 97.83 55.025) (width 0.2) (layer "B.Cu") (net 12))
 (segment (start 130 86.5) (end 123.05 79.55) (width 0.2) (layer "B.Cu") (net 12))
 (segment (start 140.5975 88.4375) (end 138.66 86.5) (width 0.2) (layer "B.Cu") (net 12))
 (segment (start 138.66 86.5) (end 130 86.5) (width 0.2) (layer "B.Cu") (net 12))
 (segment (start 135.302 57.625) (end 135.302 54.625) (width 0.2) (layer "B.Cu") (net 12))
 (segment (start 123.05 62.125) (end 123.15 62.025) (width 0.2) (layer "B.Cu") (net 12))
 (segment (start 134.55 57.625) (end 135.302 57.625) (width 0.2) (layer "B.Cu") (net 12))
 (segment (start 123.05 79.55) (end 123.05 62.125) (width 0.2) (layer "B.Cu") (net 12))
 (segment (start 135.302 54.625) (end 98.23 54.625) (width 0.2) (layer "B.Cu") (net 12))
 (segment (start 130.15 62.025) (end 134.55 57.625) (width 0.2) (layer "B.Cu") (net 12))
 (segment (start 123.15 62.025) (end 130.15 62.025) (width 0.2) (layer "B.Cu") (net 12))
 (segment (start 97.83 55.025) (end 97.83 65.185) (width 0.2) (layer "B.Cu") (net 12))
 (segment (start 97.83 65.185) (end 98.93 66.285) (width 0.2) (layer "B.Cu") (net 12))
 (segment (start 101.59 99.46) (end 101.59 95.125) (width 0.2) (layer "B.Cu") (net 16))
 (segment (start 112.067818 65.847182) (end 114.17 63.745) (width 0.2) (layer "B.Cu") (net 16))
 (segment (start 112.067818 72.642818) (end 112.067818 65.847182) (width 0.2) (layer "B.Cu") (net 16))
 (segment (start 101.59 118.51) (end 101.59 99.46) (width 0.2) (layer "B.Cu") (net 16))
 (segment (start 101.59 95.125) (end 113.05 95.125) (width 0.2) (layer "B.Cu") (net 16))
 (segment (start 113.05 95.125) (end 119.35 88.825) (width 0.2) (layer "B.Cu") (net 16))
 (segment (start 119.35 78.240686) (end 115.034314 73.925) (width 0.2) (layer "B.Cu") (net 16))
 (segment (start 115.034314 73.925) (end 113.35 73.925) (width 0.2) (layer "B.Cu") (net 16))
 (segment (start 119.35 88.825) (end 119.35 78.240686) (width 0.2) (layer "B.Cu") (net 16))
 (segment (start 113.35 73.925) (end 112.067818 72.642818) (width 0.2) (layer "B.Cu") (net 16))
 (segment (start 120.64 118.51) (end 120.64 99.46) (width 0.2) (layer "B.Cu") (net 3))
 (segment (start 115.2 73.525) (end 113.515686 73.525) (width 0.2) (layer "B.Cu") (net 3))
 (segment (start 112.467818 72.477132) (end 112.467818 67.987182) (width 0.2) (layer "B.Cu") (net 3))
 (segment (start 112.467818 67.987182) (end 114.17 66.285) (width 0.2) (layer "B.Cu") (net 3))
 (segment (start 119.75 98.57) (end 119.75 78.075) (width 0.2) (layer "B.Cu") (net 3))
 (segment (start 113.515686 73.525) (end 112.467818 72.477132) (width 0.2) (layer "B.Cu") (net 3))
 (segment (start 119.75 78.075) (end 115.2 73.525) (width 0.2) (layer "B.Cu") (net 3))
 (segment (start 120.64 99.46) (end 119.75 98.57) (width 0.2) (layer "B.Cu") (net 3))
 (segment (start 122.55 99.125) (end 128.05 99.125) (width 0.2) (layer "B.Cu") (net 5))
 (segment (start 120.15 77.909314) (end 120.15 96.725) (width 0.2) (layer "B.Cu") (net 5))
 (segment (start 120.15 96.725) (end 122.55 99.125) (width 0.2) (layer "B.Cu") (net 5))
 (segment (start 150.5 104.5) (end 150.55 104.55) (width 0.2) (layer "B.Cu") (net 5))
 (segment (start 115.365685 73.125) (end 115.8 73.559315) (width 0.2) (layer "B.Cu") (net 5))
 (segment (start 112.867818 72.311446) (end 113.681372 73.125) (width 0.2) (layer "B.Cu") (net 5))
 (segment (start 150.55 104.55) (end 150.55 107.65) (width 0.2) (layer "B.Cu") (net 5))
 (segment (start 128.05 99.125) (end 128.05 105.8) (width 0.2) (layer "B.Cu") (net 5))
 (segment (start 115.8 73.559315) (end 120.15 77.909314) (width 0.2) (layer "B.Cu") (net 5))
 (segment (start 114.17 68.825) (end 112.867818 70.127182) (width 0.2) (layer "B.Cu") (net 5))
 (segment (start 113.681372 73.125) (end 115.365685 73.125) (width 0.2) (layer "B.Cu") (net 5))
 (segment (start 150.55 107.65) (end 139.69 118.51) (width 0.2) (layer "B.Cu") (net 5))
 (segment (start 149.2 105.8) (end 150.5 104.5) (width 0.2) (layer "B.Cu") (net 5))
 (segment (start 112.867818 70.127182) (end 112.867818 72.311446) (width 0.2) (layer "B.Cu") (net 5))
 (segment (start 128.05 105.8) (end 149.2 105.8) (width 0.2) (layer "B.Cu") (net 5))
 (segment (start 122.184163 84.775) (end 124.15 86.740837) (width 0.2) (layer "F.Cu") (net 13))
 (segment (start 120.7 80.007143) (end 120.7 84.775) (width 0.2) (layer "F.Cu") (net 13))
 (segment (start 134.55 103.05) (end 136 104.5) (width 0.2) (layer "F.Cu") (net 13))
 (segment (start 120.7 84.775) (end 122.184163 84.775) (width 0.2) (layer "F.Cu") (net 13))
 (segment (start 134.55 96.297092) (end 134.55 103.05) (width 0.2) (layer "F.Cu") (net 13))
 (segment (start 124.15 91.025) (end 126.55 93.425) (width 0.2) (layer "F.Cu") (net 13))
 (segment (start 101.225 74.105) (end 114.797857 74.105) (width 0.2) (layer "F.Cu") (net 13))
 (segment (start 114.797857 74.105) (end 120.7 80.007143) (width 0.2) (layer "F.Cu") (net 13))
 (segment (start 131.677908 93.425) (end 134.55 96.297092) (width 0.2) (layer "F.Cu") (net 13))
 (segment (start 124.15 86.740837) (end 124.15 91.025) (width 0.2) (layer "F.Cu") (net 13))
 (segment (start 126.55 93.425) (end 131.677908 93.425) (width 0.2) (layer "F.Cu") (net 13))
 (segment (start 98.485 71.365) (end 101.225 74.105) (width 0.2) (layer "F.Cu") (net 13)))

